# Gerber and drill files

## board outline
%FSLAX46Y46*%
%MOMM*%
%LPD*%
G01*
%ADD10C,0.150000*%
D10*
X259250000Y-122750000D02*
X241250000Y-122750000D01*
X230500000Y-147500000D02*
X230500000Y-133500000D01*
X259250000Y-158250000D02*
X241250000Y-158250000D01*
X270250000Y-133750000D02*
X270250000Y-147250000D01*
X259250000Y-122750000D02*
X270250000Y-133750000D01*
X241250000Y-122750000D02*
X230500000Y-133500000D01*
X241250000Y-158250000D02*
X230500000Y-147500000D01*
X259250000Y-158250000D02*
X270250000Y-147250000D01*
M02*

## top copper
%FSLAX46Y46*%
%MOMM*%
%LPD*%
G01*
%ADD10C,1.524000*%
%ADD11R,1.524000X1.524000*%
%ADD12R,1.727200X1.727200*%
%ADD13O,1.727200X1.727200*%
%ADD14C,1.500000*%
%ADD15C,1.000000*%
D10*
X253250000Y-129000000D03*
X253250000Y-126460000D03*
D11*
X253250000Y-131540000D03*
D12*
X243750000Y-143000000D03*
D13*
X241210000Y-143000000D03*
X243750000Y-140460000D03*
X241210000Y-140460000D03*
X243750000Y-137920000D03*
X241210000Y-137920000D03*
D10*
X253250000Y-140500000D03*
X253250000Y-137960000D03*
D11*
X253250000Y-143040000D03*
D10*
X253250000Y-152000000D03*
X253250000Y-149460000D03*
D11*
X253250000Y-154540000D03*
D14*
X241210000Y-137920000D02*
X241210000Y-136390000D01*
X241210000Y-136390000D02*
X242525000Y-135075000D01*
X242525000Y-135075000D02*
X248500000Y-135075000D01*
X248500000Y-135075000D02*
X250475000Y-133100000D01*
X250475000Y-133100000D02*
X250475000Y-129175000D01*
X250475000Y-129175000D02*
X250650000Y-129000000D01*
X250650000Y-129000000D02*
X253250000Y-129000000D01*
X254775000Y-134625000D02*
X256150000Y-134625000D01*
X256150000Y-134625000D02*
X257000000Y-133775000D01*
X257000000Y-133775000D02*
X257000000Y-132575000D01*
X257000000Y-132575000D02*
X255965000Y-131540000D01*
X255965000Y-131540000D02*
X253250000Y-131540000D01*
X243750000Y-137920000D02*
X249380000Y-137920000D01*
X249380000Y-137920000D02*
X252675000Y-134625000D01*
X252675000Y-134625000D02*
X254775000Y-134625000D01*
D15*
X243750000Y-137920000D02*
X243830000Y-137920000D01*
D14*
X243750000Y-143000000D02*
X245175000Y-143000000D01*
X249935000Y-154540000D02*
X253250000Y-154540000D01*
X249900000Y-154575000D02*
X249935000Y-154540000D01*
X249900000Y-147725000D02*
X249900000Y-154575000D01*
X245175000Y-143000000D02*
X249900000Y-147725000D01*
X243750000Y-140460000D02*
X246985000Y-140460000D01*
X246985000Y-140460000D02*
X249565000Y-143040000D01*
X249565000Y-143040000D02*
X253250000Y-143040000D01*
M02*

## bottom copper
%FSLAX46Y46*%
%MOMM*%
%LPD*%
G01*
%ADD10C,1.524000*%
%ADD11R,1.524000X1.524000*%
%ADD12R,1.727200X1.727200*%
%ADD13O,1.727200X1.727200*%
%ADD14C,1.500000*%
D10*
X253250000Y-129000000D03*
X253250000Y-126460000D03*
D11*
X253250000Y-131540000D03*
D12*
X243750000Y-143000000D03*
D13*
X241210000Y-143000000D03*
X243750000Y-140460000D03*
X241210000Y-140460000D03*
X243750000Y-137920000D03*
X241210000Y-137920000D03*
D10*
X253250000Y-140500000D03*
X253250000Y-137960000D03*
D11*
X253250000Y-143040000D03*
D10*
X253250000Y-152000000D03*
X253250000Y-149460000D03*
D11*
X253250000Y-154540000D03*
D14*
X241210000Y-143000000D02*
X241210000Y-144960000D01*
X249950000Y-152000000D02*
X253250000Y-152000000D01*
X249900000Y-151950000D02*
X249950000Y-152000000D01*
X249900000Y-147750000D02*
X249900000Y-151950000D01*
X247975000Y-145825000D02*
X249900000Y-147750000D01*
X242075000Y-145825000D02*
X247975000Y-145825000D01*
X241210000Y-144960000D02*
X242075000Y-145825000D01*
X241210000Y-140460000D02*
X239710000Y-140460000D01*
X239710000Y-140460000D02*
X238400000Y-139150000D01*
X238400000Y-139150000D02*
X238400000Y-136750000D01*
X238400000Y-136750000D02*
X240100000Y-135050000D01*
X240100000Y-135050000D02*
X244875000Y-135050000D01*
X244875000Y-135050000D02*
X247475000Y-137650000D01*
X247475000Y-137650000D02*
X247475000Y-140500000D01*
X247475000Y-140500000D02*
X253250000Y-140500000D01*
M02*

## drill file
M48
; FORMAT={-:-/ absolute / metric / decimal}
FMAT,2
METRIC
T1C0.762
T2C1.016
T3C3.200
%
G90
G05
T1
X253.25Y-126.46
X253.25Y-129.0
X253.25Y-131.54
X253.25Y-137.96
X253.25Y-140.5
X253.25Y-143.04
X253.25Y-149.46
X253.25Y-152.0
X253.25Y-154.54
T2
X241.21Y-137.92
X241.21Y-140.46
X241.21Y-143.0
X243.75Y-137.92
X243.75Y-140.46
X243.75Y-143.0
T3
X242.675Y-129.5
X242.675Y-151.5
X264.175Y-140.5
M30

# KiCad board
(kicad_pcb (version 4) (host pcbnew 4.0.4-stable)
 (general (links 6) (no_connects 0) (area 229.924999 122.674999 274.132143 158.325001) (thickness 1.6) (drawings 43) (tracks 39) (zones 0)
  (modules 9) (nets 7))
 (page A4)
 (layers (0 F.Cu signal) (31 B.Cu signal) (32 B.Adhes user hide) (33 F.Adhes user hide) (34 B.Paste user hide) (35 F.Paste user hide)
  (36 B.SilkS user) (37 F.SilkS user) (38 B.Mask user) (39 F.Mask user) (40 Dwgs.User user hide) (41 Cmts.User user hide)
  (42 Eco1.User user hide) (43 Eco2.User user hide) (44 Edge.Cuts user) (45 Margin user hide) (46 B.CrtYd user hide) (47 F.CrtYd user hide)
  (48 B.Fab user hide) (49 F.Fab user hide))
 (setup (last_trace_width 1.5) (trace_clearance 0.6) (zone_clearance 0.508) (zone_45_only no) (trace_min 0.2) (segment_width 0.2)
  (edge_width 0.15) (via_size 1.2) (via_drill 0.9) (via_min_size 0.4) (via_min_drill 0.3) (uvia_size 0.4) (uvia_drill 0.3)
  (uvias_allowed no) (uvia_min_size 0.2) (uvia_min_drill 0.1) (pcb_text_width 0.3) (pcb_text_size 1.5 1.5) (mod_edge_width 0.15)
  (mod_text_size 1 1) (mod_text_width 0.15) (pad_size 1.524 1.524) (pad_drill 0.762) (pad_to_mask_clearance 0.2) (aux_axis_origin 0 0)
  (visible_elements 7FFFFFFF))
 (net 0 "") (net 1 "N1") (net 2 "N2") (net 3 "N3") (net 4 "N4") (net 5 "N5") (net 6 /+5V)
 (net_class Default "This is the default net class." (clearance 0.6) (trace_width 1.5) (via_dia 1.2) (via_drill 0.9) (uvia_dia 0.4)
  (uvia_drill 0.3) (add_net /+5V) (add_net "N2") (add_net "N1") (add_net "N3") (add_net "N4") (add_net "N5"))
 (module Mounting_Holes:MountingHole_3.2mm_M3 (layer F.Cu) (at 264.175 140.5)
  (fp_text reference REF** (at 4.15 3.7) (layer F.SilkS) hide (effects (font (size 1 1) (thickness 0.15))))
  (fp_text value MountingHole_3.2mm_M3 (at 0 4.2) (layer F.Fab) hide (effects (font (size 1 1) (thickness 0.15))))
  (pad 1 np_thru_hole circle (at 0 0) (size 3.2 3.2) (drill 3.2) (layers *.Cu *.Mask)))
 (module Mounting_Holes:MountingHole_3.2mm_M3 (layer F.Cu) (at 242.675 151.5)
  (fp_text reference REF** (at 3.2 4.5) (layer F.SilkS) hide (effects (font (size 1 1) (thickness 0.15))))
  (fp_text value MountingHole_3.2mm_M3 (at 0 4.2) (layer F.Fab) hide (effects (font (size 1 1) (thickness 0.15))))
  (pad 1 np_thru_hole circle (at 0 0) (size 3.2 3.2) (drill 3.2) (layers *.Cu *.Mask)))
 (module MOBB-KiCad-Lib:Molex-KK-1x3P (layer B.Cu) (at 253.25 129 270)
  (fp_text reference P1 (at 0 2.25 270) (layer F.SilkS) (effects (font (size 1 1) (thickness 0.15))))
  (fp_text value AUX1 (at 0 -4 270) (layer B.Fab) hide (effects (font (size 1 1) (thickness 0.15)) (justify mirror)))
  (pad 2 thru_hole circle (at 0 0 270) (size 1.524 1.524) (drill 0.762) (layers *.Cu *.Mask) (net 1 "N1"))
  (pad 3 thru_hole circle (at -2.54 0 270) (size 1.524 1.524) (drill 0.762) (layers *.Cu *.Mask))
  (pad 1 thru_hole rect (at 2.54 0 270) (size 1.524 1.524) (drill 0.762) (layers *.Cu *.Mask) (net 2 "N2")))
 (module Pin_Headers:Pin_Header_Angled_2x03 (layer F.Cu) (at 243.75 143 180)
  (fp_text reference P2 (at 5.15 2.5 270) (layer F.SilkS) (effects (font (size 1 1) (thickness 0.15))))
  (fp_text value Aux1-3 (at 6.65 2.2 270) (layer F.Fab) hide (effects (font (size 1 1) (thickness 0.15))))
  (pad 1 thru_hole rect (at 0 0 180) (size 1.7272 1.7272) (drill 1.016) (layers *.Cu *.Mask) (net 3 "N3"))
  (pad 2 thru_hole oval (at 2.54 0 180) (size 1.7272 1.7272) (drill 1.016) (layers *.Cu *.Mask) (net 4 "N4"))
  (pad 3 thru_hole oval (at 0 2.54 180) (size 1.7272 1.7272) (drill 1.016) (layers *.Cu *.Mask) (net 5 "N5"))
  (pad 4 thru_hole oval (at 2.54 2.54 180) (size 1.7272 1.7272) (drill 1.016) (layers *.Cu *.Mask) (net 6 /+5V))
  (pad 5 thru_hole oval (at 0 5.08 180) (size 1.7272 1.7272) (drill 1.016) (layers *.Cu *.Mask) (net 2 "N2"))
  (pad 6 thru_hole oval (at 2.54 5.08 180) (size 1.7272 1.7272) (drill 1.016) (layers *.Cu *.Mask) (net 1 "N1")))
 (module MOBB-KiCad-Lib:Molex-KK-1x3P (layer B.Cu) (at 253.25 140.5 270)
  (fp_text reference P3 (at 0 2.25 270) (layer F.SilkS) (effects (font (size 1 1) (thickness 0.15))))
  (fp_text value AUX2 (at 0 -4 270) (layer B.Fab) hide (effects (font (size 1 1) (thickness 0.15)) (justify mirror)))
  (pad 2 thru_hole circle (at 0 0 270) (size 1.524 1.524) (drill 0.762) (layers *.Cu *.Mask) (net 6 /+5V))
  (pad 3 thru_hole circle (at -2.54 0 270) (size 1.524 1.524) (drill 0.762) (layers *.Cu *.Mask))
  (pad 1 thru_hole rect (at 2.54 0 270) (size 1.524 1.524) (drill 0.762) (layers *.Cu *.Mask) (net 5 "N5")))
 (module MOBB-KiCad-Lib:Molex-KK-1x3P (layer B.Cu) (at 253.25 152 270)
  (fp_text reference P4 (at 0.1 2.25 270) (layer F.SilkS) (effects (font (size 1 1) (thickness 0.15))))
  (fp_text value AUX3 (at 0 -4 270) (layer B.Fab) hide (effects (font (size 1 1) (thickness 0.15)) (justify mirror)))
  (pad 2 thru_hole circle (at 0 0 270) (size 1.524 1.524) (drill 0.762) (layers *.Cu *.Mask) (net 4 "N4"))
  (pad 3 thru_hole circle (at -2.54 0 270) (size 1.524 1.524) (drill 0.762) (layers *.Cu *.Mask))
  (pad 1 thru_hole rect (at 2.54 0 270) (size 1.524 1.524) (drill 0.762) (layers *.Cu *.Mask) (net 3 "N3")))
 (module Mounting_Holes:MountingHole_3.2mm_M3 (layer F.Cu) (at 242.675 129.5)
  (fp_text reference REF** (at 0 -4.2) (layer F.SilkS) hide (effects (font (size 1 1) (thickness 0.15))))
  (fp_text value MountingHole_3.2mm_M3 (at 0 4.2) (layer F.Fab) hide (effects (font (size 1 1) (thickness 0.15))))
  (pad 1 np_thru_hole circle (at 0 0) (size 3.2 3.2) (drill 3.2) (layers *.Cu *.Mask)))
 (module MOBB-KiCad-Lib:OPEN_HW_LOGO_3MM (layer F.Cu) (at 237.1 130.5)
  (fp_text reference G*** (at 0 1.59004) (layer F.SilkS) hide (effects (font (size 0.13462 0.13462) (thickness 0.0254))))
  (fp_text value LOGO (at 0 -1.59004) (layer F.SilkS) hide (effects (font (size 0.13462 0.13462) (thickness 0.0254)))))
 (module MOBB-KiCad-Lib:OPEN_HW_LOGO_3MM (layer B.Cu) (at 237.1 130.5 180)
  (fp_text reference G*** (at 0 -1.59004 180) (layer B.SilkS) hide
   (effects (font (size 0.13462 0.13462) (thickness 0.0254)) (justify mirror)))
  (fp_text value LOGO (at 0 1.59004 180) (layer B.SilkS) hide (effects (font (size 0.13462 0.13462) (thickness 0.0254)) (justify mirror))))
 (gr_line (start 259.25 122.75) (end 241.25 122.75) (angle 90) (layer Edge.Cuts) (width 0.15))
 (gr_line (start 230.5 147.5) (end 230.5 133.5) (angle 90) (layer Edge.Cuts) (width 0.15))
 (gr_line (start 259.25 158.25) (end 241.25 158.25) (angle 90) (layer Edge.Cuts) (width 0.15))
 (gr_line (start 270.25 133.75) (end 270.25 147.25) (angle 90) (layer Edge.Cuts) (width 0.15))
 (gr_line (start 259.25 122.75) (end 270.25 133.75) (angle 90) (layer Edge.Cuts) (width 0.15))
 (gr_line (start 241.25 122.75) (end 230.5 133.5) (angle 90) (layer Edge.Cuts) (width 0.15))
 (gr_line (start 241.25 158.25) (end 230.5 147.5) (angle 90) (layer Edge.Cuts) (width 0.15))
 (gr_line (start 259.25 158.25) (end 270.25 147.25) (angle 90) (layer Edge.Cuts) (width 0.15))
 (segment (start 241.21 137.92) (end 241.21 136.39) (width 1.5) (layer F.Cu) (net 1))
 (segment (start 241.21 136.39) (end 242.525 135.075) (width 1.5) (layer F.Cu) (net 1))
 (segment (start 242.525 135.075) (end 248.5 135.075) (width 1.5) (layer F.Cu) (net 1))
 (segment (start 248.5 135.075) (end 250.475 133.1) (width 1.5) (layer F.Cu) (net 1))
 (segment (start 250.475 133.1) (end 250.475 129.175) (width 1.5) (layer F.Cu) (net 1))
 (segment (start 250.475 129.175) (end 250.65 129) (width 1.5) (layer F.Cu) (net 1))
 (segment (start 250.65 129) (end 253.25 129) (width 1.5) (layer F.Cu) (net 1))
 (segment (start 254.775 134.625) (end 256.15 134.625) (width 1.5) (layer F.Cu) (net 2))
 (segment (start 256.15 134.625) (end 257 133.775) (width 1.5) (layer F.Cu) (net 2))
 (segment (start 257 133.775) (end 257 132.575) (width 1.5) (layer F.Cu) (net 2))
 (segment (start 257 132.575) (end 255.965 131.54) (width 1.5) (layer F.Cu) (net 2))
 (segment (start 255.965 131.54) (end 253.25 131.54) (width 1.5) (layer F.Cu) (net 2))
 (segment (start 243.75 137.92) (end 249.38 137.92) (width 1.5) (layer F.Cu) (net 2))
 (segment (start 249.38 137.92) (end 252.675 134.625) (width 1.5) (layer F.Cu) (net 2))
 (segment (start 252.675 134.625) (end 254.775 134.625) (width 1.5) (layer F.Cu) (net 2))
 (segment (start 243.75 137.92) (end 243.83 137.92) (width 1) (layer F.Cu) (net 2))
 (segment (start 243.75 143) (end 245.175 143) (width 1.5) (layer F.Cu) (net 3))
 (segment (start 249.935 154.54) (end 253.25 154.54) (width 1.5) (layer F.Cu) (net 3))
 (segment (start 249.9 154.575) (end 249.935 154.54) (width 1.5) (layer F.Cu) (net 3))
 (segment (start 249.9 147.725) (end 249.9 154.575) (width 1.5) (layer F.Cu) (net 3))
 (segment (start 245.175 143) (end 249.9 147.725) (width 1.5) (layer F.Cu) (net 3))
 (segment (start 241.21 143) (end 241.21 144.96) (width 1.5) (layer B.Cu) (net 4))
 (segment (start 249.95 152) (end 253.25 152) (width 1.5) (layer B.Cu) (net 4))
 (segment (start 249.9 151.95) (end 249.95 152) (width 1.5) (layer B.Cu) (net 4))
 (segment (start 249.9 147.75) (end 249.9 151.95) (width 1.5) (layer B.Cu) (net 4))
 (segment (start 247.975 145.825) (end 249.9 147.75) (width 1.5) (layer B.Cu) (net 4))
 (segment (start 242.075 145.825) (end 247.975 145.825) (width 1.5) (layer B.Cu) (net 4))
 (segment (start 241.21 144.96) (end 242.075 145.825) (width 1.5) (layer B.Cu) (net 4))
 (segment (start 243.75 140.46) (end 246.985 140.46) (width 1.5) (layer F.Cu) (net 5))
 (segment (start 246.985 140.46) (end 249.565 143.04) (width 1.5) (layer F.Cu) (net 5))
 (segment (start 249.565 143.04) (end 253.25 143.04) (width 1.5) (layer F.Cu) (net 5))
 (segment (start 241.21 140.46) (end 239.71 140.46) (width 1.5) (layer B.Cu) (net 6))
 (segment (start 239.71 140.46) (end 238.4 139.15) (width 1.5) (layer B.Cu) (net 6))
 (segment (start 238.4 139.15) (end 238.4 136.75) (width 1.5) (layer B.Cu) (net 6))
 (segment (start 238.4 136.75) (end 240.1 135.05) (width 1.5) (layer B.Cu) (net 6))
 (segment (start 240.1 135.05) (end 244.875 135.05) (width 1.5) (layer B.Cu) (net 6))
 (segment (start 244.875 135.05) (end 247.475 137.65) (width 1.5) (layer B.Cu) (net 6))
 (segment (start 247.475 137.65) (end 247.475 140.5) (width 1.5) (layer B.Cu) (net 6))
 (segment (start 247.475 140.5) (end 253.25 140.5) (width 1.5) (layer B.Cu) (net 6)))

